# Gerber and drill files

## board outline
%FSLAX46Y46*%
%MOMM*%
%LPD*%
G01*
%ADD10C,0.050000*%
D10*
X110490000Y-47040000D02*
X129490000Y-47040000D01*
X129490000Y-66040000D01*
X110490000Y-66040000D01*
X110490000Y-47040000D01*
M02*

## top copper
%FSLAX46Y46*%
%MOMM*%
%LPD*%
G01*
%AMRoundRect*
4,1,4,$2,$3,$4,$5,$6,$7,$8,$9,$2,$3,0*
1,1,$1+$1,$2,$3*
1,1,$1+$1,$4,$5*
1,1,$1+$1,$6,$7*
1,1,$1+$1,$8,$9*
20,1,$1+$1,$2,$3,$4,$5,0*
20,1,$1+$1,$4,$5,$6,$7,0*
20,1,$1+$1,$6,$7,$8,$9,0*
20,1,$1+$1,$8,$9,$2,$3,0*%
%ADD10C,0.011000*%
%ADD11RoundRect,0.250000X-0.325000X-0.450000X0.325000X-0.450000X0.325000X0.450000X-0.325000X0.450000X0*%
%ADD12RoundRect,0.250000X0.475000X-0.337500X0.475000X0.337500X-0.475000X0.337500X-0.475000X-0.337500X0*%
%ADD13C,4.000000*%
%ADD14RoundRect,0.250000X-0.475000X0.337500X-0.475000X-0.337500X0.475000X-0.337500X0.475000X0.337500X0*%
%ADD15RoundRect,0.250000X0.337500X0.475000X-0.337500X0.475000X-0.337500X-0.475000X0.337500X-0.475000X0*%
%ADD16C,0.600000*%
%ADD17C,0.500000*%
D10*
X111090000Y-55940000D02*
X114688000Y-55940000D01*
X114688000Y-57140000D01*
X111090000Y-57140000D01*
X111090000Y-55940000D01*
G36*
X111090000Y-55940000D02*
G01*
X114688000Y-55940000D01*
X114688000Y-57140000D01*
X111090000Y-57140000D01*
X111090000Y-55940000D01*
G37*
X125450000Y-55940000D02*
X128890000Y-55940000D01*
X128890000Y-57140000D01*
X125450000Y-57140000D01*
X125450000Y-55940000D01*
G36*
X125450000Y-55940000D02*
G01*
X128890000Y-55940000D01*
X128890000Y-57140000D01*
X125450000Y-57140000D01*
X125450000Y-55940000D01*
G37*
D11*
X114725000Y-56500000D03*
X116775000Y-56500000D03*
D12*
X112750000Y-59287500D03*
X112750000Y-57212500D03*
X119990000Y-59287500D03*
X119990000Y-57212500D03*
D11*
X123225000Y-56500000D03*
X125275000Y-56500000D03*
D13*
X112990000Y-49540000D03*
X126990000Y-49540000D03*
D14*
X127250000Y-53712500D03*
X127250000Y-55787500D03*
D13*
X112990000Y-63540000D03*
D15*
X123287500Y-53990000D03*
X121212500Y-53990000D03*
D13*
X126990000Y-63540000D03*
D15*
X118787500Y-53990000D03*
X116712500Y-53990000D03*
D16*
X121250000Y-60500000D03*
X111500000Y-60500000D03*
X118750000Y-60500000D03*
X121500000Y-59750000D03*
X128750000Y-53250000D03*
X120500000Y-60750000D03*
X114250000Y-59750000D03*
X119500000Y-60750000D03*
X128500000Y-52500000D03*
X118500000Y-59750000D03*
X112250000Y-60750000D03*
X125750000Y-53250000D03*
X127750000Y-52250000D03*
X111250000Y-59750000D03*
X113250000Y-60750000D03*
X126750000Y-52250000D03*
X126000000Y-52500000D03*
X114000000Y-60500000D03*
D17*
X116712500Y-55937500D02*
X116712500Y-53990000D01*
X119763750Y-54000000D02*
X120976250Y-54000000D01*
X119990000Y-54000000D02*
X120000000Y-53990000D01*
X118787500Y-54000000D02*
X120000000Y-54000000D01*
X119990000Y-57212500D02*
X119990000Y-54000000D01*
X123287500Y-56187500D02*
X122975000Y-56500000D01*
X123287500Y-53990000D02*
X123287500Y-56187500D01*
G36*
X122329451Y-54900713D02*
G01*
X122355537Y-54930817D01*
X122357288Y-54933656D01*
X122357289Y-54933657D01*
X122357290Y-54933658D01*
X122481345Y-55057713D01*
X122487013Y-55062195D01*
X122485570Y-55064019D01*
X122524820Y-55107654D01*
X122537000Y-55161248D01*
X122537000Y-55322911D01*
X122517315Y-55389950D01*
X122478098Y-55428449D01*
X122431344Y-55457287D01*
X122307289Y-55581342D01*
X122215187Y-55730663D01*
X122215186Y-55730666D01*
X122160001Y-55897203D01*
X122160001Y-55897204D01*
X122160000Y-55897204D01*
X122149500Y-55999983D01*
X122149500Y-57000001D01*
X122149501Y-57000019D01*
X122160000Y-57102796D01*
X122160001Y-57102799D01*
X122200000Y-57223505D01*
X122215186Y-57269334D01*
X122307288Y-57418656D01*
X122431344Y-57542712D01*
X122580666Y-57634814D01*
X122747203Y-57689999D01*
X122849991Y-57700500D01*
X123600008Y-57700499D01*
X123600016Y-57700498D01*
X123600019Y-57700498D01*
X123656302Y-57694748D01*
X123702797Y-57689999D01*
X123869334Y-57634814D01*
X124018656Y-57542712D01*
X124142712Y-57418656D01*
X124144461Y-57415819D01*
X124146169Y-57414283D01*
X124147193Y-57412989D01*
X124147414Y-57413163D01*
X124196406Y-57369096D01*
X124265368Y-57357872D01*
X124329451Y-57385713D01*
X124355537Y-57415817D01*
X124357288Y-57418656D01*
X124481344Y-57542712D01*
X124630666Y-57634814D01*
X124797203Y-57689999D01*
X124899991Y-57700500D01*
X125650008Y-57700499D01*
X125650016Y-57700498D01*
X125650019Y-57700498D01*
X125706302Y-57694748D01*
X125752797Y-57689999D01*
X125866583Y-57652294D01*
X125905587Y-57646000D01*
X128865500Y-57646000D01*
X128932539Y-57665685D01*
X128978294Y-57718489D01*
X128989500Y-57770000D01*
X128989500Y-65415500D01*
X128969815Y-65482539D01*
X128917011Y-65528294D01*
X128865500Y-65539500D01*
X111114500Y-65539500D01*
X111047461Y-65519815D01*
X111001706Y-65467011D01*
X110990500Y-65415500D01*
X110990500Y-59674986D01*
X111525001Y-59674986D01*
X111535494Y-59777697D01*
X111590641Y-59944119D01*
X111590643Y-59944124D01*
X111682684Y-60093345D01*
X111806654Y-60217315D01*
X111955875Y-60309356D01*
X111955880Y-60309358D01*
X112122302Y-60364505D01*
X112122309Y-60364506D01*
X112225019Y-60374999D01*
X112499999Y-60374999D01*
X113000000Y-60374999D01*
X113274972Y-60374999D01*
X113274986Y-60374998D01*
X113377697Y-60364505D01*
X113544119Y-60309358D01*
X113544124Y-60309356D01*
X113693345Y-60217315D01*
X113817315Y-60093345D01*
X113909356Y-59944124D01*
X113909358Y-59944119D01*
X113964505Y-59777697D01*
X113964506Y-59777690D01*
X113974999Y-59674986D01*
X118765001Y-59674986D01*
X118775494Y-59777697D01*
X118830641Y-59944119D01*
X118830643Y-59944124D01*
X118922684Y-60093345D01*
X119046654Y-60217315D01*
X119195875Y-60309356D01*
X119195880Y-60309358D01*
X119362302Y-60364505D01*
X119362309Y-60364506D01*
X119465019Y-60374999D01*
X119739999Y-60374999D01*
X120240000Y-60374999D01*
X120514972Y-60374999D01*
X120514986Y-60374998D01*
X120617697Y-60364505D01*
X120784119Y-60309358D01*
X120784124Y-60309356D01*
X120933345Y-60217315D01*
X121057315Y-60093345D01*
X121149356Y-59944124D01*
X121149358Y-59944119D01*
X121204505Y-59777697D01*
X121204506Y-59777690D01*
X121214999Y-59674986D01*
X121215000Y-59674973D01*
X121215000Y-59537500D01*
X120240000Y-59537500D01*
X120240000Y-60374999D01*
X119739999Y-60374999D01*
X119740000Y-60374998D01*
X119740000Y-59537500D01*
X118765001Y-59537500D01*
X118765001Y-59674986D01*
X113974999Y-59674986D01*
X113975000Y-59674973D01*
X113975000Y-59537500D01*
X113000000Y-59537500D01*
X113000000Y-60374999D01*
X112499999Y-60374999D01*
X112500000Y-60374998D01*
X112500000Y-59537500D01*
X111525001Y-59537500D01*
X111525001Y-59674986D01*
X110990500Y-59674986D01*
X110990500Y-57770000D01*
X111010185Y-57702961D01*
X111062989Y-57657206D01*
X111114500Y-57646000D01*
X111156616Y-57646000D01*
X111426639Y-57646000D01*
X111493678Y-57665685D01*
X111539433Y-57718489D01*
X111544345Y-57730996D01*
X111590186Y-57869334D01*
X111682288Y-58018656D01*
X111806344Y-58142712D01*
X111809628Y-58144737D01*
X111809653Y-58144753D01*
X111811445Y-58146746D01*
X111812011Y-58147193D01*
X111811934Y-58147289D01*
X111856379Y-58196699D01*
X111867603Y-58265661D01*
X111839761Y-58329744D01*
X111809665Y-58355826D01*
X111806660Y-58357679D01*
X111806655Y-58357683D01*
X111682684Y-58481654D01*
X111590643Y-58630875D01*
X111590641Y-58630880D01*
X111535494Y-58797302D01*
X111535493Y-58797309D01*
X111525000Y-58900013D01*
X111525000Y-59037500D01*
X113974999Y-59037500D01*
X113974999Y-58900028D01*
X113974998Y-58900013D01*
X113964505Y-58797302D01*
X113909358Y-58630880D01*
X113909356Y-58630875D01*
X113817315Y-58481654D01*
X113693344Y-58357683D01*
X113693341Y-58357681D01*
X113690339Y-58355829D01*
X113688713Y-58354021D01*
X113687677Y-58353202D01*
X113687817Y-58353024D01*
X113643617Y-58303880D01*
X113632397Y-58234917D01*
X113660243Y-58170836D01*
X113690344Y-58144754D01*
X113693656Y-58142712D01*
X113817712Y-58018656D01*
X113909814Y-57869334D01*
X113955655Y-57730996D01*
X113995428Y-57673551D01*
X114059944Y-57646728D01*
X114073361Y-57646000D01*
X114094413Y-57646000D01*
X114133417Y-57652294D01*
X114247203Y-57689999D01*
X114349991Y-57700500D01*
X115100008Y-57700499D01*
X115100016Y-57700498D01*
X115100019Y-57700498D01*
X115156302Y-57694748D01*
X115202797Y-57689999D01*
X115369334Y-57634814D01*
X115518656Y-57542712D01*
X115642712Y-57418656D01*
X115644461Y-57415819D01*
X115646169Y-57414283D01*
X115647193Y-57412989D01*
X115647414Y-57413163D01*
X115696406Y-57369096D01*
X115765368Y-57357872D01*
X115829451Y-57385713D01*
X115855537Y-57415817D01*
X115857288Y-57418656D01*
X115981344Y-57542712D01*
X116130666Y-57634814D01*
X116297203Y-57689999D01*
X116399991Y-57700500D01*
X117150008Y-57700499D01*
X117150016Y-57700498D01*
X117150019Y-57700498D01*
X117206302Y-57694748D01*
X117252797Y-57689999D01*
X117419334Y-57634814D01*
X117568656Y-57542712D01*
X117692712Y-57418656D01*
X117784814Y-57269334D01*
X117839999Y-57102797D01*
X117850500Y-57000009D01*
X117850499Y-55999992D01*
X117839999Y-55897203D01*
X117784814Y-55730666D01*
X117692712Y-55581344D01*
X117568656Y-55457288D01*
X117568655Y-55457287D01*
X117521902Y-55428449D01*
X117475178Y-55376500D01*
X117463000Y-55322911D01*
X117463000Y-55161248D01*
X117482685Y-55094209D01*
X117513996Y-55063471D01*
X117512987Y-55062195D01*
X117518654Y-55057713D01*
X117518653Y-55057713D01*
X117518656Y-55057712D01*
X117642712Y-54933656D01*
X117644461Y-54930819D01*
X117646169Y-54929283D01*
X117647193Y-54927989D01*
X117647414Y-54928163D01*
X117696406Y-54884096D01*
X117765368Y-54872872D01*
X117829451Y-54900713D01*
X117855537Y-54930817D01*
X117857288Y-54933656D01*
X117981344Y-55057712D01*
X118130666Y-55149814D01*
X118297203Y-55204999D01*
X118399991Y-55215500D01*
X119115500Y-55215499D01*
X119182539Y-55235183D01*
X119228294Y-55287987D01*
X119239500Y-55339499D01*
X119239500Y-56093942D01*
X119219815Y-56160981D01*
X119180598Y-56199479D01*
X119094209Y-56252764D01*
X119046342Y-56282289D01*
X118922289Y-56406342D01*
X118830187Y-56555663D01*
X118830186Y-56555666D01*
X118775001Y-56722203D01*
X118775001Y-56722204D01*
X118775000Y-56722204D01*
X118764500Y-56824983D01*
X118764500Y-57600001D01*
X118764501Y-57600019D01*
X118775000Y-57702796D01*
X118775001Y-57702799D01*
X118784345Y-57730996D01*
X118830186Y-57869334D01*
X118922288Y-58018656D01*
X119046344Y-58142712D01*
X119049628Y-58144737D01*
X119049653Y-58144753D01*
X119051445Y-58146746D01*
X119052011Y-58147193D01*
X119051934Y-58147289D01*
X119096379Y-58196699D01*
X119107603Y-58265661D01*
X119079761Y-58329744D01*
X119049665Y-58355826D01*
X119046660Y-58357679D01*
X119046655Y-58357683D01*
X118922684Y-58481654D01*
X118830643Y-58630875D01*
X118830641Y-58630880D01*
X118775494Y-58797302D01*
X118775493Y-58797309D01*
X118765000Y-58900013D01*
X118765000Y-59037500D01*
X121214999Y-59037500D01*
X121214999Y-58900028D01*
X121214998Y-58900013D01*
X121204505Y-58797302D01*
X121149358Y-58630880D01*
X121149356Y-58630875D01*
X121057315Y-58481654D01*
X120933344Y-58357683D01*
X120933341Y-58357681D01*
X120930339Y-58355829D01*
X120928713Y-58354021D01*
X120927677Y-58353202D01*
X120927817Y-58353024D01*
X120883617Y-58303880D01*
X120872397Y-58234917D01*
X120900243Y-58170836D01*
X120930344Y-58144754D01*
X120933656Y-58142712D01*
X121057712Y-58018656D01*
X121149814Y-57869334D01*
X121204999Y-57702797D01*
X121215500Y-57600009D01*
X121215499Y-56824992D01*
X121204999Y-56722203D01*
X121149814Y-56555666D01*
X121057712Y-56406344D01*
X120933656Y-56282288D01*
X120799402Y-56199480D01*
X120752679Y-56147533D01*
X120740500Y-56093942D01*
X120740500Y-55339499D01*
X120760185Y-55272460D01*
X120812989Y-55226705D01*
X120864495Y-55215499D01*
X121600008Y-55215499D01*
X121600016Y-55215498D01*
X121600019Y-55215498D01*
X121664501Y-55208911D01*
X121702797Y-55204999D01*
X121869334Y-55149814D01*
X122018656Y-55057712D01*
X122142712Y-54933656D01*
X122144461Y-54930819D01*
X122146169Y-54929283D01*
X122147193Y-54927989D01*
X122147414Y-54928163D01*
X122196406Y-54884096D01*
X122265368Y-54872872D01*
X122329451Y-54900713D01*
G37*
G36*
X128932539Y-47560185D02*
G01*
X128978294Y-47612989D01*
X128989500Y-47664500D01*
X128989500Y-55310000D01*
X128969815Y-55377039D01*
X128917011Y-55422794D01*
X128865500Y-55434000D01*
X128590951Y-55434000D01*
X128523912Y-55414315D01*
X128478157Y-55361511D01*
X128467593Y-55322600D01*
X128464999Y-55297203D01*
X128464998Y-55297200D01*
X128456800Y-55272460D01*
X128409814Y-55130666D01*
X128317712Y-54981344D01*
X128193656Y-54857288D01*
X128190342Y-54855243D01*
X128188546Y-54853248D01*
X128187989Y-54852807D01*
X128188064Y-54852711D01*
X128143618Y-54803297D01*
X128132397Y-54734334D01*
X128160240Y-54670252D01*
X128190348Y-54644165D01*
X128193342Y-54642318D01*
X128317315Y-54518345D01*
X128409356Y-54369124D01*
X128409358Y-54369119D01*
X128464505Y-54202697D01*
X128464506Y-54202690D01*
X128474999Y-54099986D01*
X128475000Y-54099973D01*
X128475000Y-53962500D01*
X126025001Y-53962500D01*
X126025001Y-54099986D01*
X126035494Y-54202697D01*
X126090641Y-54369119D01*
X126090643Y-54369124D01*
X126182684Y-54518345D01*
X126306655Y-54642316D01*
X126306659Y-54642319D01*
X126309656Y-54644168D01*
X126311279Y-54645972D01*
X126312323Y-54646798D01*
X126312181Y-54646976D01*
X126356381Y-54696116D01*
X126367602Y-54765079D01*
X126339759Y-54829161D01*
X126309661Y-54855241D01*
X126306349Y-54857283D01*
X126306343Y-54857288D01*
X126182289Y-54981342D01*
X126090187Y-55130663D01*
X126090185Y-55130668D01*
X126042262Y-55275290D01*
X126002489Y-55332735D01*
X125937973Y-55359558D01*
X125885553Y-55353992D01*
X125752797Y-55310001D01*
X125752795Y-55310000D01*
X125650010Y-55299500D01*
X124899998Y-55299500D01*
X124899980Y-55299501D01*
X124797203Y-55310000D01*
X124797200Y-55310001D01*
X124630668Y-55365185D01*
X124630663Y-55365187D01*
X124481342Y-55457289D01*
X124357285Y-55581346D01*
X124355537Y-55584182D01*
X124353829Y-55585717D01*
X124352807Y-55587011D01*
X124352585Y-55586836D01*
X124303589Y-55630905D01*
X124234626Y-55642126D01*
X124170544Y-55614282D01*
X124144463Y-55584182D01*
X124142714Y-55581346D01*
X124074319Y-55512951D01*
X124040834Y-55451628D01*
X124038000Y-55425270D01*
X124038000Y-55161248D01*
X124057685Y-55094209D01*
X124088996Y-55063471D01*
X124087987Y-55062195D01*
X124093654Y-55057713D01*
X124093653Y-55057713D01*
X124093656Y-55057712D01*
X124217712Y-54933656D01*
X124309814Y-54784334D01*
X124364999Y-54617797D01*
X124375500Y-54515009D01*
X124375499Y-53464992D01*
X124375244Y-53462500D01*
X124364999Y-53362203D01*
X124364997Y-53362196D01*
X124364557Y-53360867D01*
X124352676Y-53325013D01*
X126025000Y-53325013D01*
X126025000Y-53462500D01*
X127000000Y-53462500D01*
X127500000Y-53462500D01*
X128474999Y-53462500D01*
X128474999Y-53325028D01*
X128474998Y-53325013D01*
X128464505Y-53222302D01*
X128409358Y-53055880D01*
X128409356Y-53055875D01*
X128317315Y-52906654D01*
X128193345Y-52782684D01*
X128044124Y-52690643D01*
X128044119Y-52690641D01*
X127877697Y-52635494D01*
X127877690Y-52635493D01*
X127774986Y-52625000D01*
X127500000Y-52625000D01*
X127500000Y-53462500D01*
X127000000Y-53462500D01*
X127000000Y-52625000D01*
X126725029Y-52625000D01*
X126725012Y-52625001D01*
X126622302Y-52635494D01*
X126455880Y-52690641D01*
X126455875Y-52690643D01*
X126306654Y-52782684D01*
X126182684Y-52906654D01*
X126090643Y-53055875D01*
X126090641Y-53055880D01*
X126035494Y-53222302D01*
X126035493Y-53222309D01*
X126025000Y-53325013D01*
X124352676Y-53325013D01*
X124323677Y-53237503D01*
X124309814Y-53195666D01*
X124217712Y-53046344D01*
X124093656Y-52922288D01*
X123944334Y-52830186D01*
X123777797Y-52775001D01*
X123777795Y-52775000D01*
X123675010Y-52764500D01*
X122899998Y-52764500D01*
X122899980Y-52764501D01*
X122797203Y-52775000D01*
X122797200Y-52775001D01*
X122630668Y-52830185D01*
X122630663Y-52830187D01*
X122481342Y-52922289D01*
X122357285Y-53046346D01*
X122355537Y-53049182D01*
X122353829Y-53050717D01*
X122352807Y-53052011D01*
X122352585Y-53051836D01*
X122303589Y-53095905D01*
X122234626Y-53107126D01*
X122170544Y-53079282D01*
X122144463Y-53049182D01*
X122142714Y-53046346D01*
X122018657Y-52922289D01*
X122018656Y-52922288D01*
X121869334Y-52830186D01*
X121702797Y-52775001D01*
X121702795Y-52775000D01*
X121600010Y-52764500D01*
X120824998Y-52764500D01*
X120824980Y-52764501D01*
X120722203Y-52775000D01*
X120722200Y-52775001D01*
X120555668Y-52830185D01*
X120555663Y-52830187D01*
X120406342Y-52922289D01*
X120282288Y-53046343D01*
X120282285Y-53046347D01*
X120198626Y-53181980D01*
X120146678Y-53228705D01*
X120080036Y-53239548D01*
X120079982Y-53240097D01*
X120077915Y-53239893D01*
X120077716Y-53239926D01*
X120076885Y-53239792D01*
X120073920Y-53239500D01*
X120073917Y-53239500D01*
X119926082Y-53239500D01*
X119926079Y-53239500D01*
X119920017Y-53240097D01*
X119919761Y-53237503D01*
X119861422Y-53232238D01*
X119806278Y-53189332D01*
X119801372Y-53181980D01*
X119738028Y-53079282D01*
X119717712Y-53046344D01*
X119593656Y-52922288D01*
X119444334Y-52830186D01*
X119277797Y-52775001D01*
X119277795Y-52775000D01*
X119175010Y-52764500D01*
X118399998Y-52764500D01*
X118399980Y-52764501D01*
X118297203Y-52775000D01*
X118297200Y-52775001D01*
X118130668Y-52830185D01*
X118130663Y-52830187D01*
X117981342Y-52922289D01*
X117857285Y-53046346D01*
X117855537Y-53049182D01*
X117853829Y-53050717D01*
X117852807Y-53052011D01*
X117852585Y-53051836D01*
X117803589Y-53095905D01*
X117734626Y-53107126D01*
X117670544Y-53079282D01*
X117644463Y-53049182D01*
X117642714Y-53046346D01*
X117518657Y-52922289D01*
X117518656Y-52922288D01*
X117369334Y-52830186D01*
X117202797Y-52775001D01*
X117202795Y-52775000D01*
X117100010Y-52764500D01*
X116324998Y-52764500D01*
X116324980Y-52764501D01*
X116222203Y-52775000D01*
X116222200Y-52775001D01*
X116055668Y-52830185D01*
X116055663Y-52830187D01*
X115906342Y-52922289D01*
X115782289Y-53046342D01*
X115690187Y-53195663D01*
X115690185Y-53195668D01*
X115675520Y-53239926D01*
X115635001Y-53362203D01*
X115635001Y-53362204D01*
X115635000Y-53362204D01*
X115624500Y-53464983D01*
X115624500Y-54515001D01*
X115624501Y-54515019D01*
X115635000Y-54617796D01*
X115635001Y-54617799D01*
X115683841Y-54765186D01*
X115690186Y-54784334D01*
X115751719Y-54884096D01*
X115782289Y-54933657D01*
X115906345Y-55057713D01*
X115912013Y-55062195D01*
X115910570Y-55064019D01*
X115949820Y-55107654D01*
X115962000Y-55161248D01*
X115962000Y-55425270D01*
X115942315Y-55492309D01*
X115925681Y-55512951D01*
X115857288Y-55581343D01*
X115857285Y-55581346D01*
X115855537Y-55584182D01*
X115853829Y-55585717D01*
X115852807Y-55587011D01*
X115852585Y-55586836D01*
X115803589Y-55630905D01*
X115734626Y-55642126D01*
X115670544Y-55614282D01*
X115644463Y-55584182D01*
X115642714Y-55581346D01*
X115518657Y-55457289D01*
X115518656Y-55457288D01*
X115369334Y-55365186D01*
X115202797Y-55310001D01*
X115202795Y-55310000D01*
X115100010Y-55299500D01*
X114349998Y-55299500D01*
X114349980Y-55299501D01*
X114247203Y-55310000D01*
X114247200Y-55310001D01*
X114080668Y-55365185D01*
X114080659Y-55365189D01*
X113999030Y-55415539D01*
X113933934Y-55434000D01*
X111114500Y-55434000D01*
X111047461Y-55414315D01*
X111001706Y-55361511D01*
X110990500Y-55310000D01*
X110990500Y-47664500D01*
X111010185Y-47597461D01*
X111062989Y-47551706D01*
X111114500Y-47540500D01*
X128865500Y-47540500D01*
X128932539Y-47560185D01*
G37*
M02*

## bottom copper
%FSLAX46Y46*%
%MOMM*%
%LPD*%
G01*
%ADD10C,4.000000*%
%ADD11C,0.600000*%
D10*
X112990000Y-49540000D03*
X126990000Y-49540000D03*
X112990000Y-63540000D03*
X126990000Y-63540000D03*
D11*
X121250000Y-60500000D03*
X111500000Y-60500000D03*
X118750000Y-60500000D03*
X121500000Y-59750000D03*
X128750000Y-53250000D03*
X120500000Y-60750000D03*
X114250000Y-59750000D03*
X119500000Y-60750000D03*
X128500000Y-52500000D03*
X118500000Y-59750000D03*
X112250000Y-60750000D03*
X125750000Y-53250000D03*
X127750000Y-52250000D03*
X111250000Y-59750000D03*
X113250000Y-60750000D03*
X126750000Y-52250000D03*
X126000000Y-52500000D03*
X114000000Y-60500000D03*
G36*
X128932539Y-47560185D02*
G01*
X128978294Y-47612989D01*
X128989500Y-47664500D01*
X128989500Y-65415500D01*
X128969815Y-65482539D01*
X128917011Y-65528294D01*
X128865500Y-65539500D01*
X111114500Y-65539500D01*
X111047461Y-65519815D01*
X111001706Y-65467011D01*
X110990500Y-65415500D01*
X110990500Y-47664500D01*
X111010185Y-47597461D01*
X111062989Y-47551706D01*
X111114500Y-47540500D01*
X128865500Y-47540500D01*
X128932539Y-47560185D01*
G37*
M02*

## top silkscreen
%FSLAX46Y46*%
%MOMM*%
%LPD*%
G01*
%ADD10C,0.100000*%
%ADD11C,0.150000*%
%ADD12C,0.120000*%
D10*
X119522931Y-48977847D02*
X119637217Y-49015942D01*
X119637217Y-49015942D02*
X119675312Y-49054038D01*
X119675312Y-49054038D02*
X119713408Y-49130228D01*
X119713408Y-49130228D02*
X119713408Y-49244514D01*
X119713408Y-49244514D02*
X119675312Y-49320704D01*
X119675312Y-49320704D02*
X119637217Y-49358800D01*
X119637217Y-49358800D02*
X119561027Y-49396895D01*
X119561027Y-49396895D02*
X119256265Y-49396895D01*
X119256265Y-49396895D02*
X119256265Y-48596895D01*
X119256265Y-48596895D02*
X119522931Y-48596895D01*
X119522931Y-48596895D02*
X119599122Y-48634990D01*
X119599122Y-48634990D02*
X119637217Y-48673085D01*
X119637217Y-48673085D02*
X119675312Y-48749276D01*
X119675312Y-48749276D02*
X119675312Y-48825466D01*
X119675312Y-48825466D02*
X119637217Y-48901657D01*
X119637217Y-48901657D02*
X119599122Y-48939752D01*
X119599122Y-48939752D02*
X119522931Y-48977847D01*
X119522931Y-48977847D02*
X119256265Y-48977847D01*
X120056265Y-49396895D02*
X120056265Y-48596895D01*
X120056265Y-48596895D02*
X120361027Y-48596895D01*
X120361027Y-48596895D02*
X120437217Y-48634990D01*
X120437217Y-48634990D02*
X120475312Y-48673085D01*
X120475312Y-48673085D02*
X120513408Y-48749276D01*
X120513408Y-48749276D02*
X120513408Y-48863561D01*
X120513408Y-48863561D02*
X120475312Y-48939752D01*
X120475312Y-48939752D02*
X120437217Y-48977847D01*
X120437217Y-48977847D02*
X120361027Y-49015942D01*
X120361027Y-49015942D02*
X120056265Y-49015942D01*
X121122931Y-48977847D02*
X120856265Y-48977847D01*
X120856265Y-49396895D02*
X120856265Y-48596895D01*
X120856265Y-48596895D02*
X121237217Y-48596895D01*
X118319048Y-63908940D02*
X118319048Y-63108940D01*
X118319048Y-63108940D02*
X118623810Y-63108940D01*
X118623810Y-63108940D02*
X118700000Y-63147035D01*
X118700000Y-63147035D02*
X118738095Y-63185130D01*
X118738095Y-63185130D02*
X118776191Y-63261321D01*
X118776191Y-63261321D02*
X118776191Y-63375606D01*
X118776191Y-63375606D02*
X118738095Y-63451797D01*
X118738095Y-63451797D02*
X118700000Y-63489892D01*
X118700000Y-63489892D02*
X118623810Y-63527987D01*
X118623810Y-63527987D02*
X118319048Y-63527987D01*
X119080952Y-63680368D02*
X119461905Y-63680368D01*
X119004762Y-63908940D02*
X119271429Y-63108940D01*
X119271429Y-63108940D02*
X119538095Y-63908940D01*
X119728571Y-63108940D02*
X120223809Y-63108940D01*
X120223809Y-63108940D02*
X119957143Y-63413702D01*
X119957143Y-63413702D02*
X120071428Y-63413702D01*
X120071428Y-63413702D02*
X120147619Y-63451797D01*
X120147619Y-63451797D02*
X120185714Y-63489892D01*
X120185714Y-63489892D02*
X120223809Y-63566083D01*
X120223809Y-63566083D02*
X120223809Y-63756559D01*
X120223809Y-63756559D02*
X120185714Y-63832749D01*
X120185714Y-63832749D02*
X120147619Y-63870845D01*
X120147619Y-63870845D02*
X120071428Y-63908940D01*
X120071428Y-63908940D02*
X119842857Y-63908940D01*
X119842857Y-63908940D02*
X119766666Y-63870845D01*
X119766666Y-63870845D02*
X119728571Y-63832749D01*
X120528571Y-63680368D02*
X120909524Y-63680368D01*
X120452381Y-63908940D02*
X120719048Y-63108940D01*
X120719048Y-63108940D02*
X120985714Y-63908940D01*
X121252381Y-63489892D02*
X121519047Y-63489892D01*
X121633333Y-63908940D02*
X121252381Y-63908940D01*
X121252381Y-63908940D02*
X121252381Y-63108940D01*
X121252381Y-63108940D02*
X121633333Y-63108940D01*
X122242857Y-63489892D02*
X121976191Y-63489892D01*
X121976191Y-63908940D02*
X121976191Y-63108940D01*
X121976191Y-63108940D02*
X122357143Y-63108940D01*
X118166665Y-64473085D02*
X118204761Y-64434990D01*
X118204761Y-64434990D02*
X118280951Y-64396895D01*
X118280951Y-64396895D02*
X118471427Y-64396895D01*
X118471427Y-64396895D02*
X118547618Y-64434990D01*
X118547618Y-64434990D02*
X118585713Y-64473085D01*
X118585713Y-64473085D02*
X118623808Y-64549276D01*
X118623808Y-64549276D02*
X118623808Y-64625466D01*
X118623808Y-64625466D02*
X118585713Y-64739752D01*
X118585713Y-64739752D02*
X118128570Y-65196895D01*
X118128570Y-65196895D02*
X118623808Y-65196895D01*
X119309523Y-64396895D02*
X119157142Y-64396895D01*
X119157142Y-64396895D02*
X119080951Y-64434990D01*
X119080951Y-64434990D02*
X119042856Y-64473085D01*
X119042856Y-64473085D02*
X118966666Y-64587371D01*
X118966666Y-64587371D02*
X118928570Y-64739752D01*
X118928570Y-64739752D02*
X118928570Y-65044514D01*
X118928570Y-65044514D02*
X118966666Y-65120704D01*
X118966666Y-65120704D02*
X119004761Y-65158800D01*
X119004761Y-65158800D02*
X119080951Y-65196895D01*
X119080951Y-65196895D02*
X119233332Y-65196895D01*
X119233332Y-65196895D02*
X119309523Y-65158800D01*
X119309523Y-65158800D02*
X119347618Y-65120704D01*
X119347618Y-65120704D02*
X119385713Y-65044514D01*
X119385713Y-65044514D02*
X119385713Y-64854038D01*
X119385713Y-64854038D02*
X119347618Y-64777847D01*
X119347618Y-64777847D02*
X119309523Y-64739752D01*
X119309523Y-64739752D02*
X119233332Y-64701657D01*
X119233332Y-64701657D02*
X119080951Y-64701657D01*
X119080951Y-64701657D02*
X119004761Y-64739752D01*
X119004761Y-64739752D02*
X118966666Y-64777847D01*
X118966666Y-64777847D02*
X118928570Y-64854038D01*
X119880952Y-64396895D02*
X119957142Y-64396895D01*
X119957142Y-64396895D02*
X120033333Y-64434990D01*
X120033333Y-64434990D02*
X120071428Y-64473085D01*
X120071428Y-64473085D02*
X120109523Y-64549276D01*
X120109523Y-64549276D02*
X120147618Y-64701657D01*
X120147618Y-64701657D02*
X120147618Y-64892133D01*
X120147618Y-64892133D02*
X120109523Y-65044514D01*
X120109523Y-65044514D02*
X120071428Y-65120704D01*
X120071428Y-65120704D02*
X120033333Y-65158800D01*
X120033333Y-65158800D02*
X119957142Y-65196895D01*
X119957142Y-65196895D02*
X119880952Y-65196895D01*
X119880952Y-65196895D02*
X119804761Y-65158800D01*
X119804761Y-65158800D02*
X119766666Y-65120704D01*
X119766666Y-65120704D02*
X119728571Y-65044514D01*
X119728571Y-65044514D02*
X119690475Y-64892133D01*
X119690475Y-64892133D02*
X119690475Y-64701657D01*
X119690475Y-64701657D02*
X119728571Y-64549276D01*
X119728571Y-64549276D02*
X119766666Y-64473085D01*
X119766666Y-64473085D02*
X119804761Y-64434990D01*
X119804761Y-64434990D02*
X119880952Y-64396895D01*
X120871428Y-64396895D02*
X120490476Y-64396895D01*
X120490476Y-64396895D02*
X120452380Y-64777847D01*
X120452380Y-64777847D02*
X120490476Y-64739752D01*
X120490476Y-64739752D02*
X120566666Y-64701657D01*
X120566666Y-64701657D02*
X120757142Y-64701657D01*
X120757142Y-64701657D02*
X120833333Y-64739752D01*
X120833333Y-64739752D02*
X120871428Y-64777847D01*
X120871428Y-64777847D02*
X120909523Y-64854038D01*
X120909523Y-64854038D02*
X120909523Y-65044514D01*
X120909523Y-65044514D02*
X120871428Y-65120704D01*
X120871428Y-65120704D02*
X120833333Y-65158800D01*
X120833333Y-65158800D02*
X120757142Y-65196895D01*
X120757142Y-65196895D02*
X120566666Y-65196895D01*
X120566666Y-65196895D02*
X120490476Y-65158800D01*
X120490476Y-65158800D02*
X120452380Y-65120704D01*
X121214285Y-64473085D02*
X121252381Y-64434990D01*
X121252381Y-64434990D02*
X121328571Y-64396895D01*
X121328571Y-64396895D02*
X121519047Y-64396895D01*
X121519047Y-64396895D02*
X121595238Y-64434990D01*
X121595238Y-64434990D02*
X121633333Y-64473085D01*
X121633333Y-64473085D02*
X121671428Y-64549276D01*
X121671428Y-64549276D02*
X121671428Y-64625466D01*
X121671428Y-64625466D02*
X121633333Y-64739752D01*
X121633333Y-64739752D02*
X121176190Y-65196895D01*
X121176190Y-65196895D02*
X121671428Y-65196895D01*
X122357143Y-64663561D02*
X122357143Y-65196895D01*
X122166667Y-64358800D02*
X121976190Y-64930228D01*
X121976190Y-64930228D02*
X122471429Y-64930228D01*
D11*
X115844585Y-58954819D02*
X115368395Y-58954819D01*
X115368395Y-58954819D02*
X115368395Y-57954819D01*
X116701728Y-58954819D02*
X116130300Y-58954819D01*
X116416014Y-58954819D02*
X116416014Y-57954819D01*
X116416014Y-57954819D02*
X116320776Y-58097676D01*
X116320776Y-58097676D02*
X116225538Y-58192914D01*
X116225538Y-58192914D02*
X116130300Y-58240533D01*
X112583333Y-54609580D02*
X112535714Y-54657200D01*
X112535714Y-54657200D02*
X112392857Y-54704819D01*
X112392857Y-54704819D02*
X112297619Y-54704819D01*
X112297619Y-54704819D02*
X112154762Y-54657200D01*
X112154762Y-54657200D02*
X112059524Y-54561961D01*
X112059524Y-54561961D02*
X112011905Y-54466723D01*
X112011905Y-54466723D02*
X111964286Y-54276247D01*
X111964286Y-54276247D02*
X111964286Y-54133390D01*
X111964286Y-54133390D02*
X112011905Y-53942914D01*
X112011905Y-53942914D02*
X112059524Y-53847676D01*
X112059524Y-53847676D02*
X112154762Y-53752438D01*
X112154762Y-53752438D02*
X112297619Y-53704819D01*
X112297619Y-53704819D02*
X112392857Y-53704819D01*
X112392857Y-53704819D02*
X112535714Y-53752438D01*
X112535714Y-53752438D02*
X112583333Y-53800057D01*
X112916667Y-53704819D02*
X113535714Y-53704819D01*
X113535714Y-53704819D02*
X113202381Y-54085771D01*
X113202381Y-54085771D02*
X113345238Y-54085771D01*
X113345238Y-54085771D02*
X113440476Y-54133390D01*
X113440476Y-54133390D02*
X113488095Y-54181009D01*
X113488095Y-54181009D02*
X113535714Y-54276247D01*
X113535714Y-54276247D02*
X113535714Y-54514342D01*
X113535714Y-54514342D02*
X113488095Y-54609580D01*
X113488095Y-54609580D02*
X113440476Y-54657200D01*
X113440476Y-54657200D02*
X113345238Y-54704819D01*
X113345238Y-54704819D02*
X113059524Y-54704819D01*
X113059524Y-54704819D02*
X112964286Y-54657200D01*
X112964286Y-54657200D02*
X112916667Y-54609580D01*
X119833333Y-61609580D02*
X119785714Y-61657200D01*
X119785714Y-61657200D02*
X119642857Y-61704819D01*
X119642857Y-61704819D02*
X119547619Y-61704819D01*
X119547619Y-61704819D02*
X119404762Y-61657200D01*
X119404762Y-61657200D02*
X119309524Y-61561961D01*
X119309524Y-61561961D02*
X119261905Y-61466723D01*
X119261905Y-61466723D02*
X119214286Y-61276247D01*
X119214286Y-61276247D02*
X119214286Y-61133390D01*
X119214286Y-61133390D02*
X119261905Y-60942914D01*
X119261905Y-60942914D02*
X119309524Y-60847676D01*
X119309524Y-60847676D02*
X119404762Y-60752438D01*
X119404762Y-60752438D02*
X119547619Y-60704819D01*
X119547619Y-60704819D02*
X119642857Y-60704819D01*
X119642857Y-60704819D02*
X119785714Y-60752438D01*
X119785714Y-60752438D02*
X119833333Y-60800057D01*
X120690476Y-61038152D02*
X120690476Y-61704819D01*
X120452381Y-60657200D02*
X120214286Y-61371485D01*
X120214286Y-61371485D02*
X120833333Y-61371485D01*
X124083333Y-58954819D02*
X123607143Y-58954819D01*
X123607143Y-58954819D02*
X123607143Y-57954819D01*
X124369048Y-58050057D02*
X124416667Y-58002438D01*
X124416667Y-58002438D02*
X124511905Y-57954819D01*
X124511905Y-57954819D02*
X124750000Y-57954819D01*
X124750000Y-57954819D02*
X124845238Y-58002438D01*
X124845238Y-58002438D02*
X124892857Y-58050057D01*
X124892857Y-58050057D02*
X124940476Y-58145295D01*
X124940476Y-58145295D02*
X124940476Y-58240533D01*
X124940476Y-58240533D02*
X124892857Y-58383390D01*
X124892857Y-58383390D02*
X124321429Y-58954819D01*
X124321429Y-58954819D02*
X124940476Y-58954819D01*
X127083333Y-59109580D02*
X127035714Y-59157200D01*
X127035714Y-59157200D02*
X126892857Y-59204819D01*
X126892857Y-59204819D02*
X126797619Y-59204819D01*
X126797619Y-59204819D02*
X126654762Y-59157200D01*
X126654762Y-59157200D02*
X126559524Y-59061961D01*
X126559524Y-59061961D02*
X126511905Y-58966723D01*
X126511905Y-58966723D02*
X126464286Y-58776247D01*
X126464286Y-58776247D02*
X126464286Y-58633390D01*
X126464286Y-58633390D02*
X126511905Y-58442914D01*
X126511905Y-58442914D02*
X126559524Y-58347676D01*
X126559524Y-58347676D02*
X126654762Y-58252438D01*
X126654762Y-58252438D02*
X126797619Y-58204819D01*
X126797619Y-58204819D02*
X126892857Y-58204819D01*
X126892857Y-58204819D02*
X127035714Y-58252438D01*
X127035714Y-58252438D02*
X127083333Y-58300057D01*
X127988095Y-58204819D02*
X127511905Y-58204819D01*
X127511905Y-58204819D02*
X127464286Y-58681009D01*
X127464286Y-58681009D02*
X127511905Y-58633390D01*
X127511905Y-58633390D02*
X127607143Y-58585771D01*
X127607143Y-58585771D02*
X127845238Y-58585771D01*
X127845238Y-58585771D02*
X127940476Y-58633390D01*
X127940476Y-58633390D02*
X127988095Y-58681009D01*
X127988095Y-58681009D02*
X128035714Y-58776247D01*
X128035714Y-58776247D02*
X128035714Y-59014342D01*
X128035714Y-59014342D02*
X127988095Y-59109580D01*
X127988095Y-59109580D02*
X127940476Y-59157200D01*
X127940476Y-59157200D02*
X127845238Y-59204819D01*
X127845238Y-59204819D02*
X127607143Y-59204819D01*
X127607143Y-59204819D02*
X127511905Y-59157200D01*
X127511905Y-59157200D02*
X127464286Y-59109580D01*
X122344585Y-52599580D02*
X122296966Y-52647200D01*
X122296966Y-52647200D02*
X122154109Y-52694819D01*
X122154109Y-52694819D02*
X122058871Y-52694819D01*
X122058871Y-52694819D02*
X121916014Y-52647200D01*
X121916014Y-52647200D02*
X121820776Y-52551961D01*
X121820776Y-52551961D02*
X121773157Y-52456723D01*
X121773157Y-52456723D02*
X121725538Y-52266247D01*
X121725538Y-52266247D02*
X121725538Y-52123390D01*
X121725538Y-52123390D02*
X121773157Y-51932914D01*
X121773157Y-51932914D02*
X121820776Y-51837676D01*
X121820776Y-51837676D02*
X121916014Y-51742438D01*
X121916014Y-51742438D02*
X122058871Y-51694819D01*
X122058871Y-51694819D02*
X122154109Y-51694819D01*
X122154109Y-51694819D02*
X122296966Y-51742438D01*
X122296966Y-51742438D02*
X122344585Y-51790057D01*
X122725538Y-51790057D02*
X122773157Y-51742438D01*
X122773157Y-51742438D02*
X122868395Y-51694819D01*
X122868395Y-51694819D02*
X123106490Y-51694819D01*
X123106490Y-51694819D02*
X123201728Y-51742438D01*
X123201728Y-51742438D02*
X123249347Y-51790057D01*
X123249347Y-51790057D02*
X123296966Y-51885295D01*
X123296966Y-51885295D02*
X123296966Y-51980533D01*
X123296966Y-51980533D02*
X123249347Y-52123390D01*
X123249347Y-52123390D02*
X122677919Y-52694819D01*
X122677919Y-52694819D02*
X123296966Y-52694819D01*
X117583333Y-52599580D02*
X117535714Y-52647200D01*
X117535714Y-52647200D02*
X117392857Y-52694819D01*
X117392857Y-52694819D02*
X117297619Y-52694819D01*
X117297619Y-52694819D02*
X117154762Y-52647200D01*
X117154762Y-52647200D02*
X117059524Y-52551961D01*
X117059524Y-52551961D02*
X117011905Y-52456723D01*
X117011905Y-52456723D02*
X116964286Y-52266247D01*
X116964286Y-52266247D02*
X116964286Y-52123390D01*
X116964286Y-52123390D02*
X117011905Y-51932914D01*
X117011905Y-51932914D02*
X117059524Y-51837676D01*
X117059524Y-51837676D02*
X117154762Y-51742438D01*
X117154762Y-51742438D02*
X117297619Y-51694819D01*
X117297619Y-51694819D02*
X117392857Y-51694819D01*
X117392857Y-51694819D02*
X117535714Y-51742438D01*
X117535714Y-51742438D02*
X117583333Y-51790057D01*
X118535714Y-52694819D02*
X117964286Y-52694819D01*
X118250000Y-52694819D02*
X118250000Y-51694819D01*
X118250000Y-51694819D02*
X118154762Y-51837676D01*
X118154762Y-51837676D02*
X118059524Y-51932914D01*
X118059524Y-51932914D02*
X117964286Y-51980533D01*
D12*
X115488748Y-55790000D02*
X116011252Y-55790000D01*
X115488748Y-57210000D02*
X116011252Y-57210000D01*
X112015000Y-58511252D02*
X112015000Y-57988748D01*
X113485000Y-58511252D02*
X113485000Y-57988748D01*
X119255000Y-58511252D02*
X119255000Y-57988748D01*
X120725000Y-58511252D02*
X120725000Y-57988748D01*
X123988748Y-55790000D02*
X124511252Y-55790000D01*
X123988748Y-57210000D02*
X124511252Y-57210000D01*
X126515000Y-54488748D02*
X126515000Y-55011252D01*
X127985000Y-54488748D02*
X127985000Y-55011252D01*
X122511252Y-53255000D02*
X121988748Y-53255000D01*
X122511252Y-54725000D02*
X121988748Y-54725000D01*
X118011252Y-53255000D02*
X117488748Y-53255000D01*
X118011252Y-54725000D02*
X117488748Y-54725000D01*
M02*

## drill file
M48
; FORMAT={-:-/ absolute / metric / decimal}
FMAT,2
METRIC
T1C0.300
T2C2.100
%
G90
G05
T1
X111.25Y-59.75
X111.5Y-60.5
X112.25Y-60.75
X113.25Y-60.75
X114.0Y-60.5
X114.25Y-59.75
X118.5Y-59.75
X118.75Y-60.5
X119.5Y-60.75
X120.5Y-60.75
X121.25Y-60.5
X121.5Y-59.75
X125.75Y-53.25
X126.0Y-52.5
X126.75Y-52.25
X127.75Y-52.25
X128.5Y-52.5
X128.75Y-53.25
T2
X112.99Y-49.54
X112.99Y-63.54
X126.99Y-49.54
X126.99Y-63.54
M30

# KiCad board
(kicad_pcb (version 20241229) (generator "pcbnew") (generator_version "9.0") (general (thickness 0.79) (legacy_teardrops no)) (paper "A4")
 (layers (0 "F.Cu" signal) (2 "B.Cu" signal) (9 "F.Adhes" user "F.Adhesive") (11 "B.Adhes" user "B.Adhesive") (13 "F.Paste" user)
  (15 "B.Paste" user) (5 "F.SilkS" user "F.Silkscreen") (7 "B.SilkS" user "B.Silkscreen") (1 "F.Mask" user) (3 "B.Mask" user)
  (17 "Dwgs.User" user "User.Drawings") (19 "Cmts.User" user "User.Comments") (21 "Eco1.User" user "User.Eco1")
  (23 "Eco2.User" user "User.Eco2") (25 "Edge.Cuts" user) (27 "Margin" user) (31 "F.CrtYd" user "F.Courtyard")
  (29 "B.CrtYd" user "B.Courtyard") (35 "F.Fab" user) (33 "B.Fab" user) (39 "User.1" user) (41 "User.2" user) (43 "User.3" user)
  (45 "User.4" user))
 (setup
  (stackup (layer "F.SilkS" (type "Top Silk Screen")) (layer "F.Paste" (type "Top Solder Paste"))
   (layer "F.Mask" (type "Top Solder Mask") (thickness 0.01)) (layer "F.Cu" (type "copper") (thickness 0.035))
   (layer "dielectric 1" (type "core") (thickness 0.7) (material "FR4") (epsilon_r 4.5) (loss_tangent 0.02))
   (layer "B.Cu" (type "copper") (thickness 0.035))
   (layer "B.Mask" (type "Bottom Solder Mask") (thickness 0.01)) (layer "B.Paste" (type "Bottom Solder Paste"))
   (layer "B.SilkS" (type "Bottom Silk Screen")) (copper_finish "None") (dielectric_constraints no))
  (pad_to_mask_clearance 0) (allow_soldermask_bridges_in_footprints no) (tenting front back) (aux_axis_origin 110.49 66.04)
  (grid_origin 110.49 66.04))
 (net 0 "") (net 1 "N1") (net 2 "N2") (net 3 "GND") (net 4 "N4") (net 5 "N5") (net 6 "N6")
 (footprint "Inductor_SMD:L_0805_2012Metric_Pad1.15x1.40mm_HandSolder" (layer "F.Cu") (at 115.75 56.5)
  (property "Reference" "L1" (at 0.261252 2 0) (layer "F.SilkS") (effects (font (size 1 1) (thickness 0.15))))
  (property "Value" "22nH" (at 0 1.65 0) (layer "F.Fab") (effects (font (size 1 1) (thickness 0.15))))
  (fp_line (start -0.261252 -0.71) (end 0.261252 -0.71) (stroke (width 0.12) (type solid)) (layer "F.SilkS"))
  (fp_line (start -0.261252 0.71) (end 0.261252 0.71) (stroke (width 0.12) (type solid)) (layer "F.SilkS"))
  (pad "1" smd roundrect (at -1.025 0) (size 1.15 1.4) (layers "F.Cu" "F.Mask" "F.Paste") (roundrect_rratio 0.217391) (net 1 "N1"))
  (pad "2" smd roundrect (at 1.025 0) (size 1.15 1.4) (layers "F.Cu" "F.Mask" "F.Paste") (roundrect_rratio 0.217391) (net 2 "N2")))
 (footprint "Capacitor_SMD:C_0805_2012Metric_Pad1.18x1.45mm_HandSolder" (layer "F.Cu") (at 112.75 58.25 90)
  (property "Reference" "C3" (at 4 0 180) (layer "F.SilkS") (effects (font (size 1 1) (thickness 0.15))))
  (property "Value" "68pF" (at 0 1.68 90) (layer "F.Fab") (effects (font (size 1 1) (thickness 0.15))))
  (fp_line (start -0.261252 -0.735) (end 0.261252 -0.735) (stroke (width 0.12) (type solid)) (layer "F.SilkS"))
  (fp_line (start -0.261252 0.735) (end 0.261252 0.735) (stroke (width 0.12) (type solid)) (layer "F.SilkS"))
  (pad "1" smd roundrect (at -1.0375 0 90) (size 1.175 1.45) (layers "F.Cu" "F.Mask" "F.Paste") (roundrect_rratio 0.212766) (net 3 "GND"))
  (pad "2" smd roundrect (at 1.0375 0 90) (size 1.175 1.45) (layers "F.Cu" "F.Mask" "F.Paste") (roundrect_rratio 0.212766) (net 1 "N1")))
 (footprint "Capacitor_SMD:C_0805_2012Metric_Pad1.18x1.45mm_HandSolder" (layer "F.Cu") (at 119.99 58.25 90)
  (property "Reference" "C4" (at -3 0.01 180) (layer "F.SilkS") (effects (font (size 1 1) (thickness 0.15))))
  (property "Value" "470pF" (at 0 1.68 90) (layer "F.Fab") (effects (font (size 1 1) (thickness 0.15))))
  (fp_line (start -0.261252 -0.735) (end 0.261252 -0.735) (stroke (width 0.12) (type solid)) (layer "F.SilkS"))
  (fp_line (start -0.261252 0.735) (end 0.261252 0.735) (stroke (width 0.12) (type solid)) (layer "F.SilkS"))
  (pad "1" smd roundrect (at -1.0375 0 90) (size 1.175 1.45) (layers "F.Cu" "F.Mask" "F.Paste") (roundrect_rratio 0.212766) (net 3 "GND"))
  (pad "2" smd roundrect (at 1.0375 0 90) (size 1.175 1.45) (layers "F.Cu" "F.Mask" "F.Paste") (roundrect_rratio 0.212766) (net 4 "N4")))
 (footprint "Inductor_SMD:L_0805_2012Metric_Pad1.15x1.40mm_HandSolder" (layer "F.Cu") (at 124.25 56.5)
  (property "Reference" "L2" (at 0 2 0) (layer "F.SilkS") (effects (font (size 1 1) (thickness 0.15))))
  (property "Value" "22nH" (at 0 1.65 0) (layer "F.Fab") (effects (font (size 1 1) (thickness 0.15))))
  (fp_line (start -0.261252 -0.71) (end 0.261252 -0.71) (stroke (width 0.12) (type solid)) (layer "F.SilkS"))
  (fp_line (start -0.261252 0.71) (end 0.261252 0.71) (stroke (width 0.12) (type solid)) (layer "F.SilkS"))
  (pad "1" smd roundrect (at -1.025 0) (size 1.15 1.4) (layers "F.Cu" "F.Mask" "F.Paste") (roundrect_rratio 0.217391) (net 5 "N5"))
  (pad "2" smd roundrect (at 1.025 0) (size 1.15 1.4) (layers "F.Cu" "F.Mask" "F.Paste") (roundrect_rratio 0.217391) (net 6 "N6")))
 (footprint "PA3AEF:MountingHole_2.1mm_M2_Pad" (layer "F.Cu") (at 112.99 49.54)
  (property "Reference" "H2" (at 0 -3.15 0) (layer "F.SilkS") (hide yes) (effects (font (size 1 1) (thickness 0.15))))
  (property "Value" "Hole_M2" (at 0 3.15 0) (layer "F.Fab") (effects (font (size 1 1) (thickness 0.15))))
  (pad "1" thru_hole circle (at 0 0) (size 4 4) (drill 2.1) (layers "*.Cu" "*.Mask") (remove_unused_layers no) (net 3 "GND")
   (zone_connect 2)))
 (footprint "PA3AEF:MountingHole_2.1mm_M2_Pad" (layer "F.Cu") (at 126.99 49.54)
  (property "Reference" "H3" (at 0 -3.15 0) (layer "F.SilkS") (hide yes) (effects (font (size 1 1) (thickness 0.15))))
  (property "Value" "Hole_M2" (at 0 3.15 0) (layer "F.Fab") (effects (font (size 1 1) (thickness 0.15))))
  (pad "1" thru_hole circle (at 0 0) (size 4 4) (drill 2.1) (layers "*.Cu" "*.Mask") (remove_unused_layers no) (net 3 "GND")
   (zone_connect 2)))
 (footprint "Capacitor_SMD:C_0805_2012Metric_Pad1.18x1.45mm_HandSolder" (layer "F.Cu") (at 127.25 54.75 -90)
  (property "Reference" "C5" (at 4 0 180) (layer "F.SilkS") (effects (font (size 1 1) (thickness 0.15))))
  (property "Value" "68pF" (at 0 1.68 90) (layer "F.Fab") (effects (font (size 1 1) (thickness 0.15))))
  (fp_line (start -0.261252 0.735) (end 0.261252 0.735) (stroke (width 0.12) (type solid)) (layer "F.SilkS"))
  (fp_line (start -0.261252 -0.735) (end 0.261252 -0.735) (stroke (width 0.12) (type solid)) (layer "F.SilkS"))
  (pad "1" smd roundrect (at -1.0375 0 270) (size 1.175 1.45) (layers "F.Cu" "F.Mask" "F.Paste") (roundrect_rratio 0.212766) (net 3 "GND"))
  (pad "2" smd roundrect (at 1.0375 0 270) (size 1.175 1.45) (layers "F.Cu" "F.Mask" "F.Paste") (roundrect_rratio 0.212766) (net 6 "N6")))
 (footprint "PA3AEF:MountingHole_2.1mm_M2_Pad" (layer "F.Cu") (at 112.99 63.54)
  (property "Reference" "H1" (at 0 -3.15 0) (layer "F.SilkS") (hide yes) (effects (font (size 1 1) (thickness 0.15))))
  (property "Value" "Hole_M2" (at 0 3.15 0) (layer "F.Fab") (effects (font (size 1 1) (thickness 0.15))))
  (pad "1" thru_hole circle (at 0 0) (size 4 4) (drill 2.1) (layers "*.Cu" "*.Mask") (remove_unused_layers no) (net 3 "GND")
   (zone_connect 2)))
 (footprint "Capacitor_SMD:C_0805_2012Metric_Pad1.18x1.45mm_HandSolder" (layer "F.Cu") (at 122.25 53.99 180)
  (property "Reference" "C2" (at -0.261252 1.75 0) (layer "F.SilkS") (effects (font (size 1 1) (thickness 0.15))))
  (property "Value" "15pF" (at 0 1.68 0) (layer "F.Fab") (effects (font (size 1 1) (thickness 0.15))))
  (fp_line (start -0.261252 0.735) (end 0.261252 0.735) (stroke (width 0.12) (type solid)) (layer "F.SilkS"))
  (fp_line (start -0.261252 -0.735) (end 0.261252 -0.735) (stroke (width 0.12) (type solid)) (layer "F.SilkS"))
  (pad "1" smd roundrect (at -1.0375 0 180) (size 1.175 1.45) (layers "F.Cu" "F.Mask" "F.Paste") (roundrect_rratio 0.212766) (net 5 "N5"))
  (pad "2" smd roundrect (at 1.0375 0 180) (size 1.175 1.45) (layers "F.Cu" "F.Mask" "F.Paste") (roundrect_rratio 0.212766) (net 4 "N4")))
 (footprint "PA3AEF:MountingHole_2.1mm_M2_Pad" (layer "F.Cu") (at 126.99 63.54)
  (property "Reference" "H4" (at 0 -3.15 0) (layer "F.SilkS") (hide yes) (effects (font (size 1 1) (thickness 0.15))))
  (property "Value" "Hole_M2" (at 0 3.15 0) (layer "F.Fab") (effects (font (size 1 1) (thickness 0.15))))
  (pad "1" thru_hole circle (at 0 0) (size 4 4) (drill 2.1) (layers "*.Cu" "*.Mask") (remove_unused_layers no) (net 3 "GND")
   (zone_connect 2)))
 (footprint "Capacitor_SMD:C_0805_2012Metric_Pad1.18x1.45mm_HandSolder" (layer "F.Cu") (at 117.75 53.99 180)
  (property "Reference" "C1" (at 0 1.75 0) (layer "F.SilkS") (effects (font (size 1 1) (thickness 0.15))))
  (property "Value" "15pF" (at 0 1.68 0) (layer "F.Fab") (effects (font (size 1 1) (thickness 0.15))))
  (fp_line (start -0.261252 0.735) (end 0.261252 0.735) (stroke (width 0.12) (type solid)) (layer "F.SilkS"))
  (fp_line (start -0.261252 -0.735) (end 0.261252 -0.735) (stroke (width 0.12) (type solid)) (layer "F.SilkS"))
  (pad "1" smd roundrect (at -1.0375 0 180) (size 1.175 1.45) (layers "F.Cu" "F.Mask" "F.Paste") (roundrect_rratio 0.212766) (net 4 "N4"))
  (pad "2" smd roundrect (at 1.0375 0 180) (size 1.175 1.45) (layers "F.Cu" "F.Mask" "F.Paste") (roundrect_rratio 0.212766) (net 2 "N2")))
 (gr_rect (start 111.09 55.94) (end 114.688 57.14) (stroke (width 0.011) (type solid)) (fill yes) (layer "F.Cu") (net 1))
 (gr_rect (start 125.45 55.94) (end 128.89 57.14) (stroke (width 0.011) (type solid)) (fill yes) (layer "F.Cu") (net 6))
 (gr_rect (start 110.49 47.04) (end 129.49 66.04) (stroke (width 0.05) (type solid)) (fill no) (layer "Edge.Cuts"))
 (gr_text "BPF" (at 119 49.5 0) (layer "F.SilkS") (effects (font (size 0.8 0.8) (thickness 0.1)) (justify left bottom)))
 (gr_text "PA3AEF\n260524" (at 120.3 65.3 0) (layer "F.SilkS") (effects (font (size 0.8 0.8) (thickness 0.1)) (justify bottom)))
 (via (at 121.25 60.5) (size 0.6) (drill 0.3) (layers "F.Cu" "B.Cu") (free yes) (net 3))
 (via (at 111.5 60.5) (size 0.6) (drill 0.3) (layers "F.Cu" "B.Cu") (free yes) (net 3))
 (via (at 118.75 60.5) (size 0.6) (drill 0.3) (layers "F.Cu" "B.Cu") (free yes) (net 3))
 (via (at 121.5 59.75) (size 0.6) (drill 0.3) (layers "F.Cu" "B.Cu") (free yes) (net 3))
 (via (at 128.75 53.25) (size 0.6) (drill 0.3) (layers "F.Cu" "B.Cu") (free yes) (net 3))
 (via (at 120.5 60.75) (size 0.6) (drill 0.3) (layers "F.Cu" "B.Cu") (free yes) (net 3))
 (via (at 114.25 59.75) (size 0.6) (drill 0.3) (layers "F.Cu" "B.Cu") (free yes) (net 3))
 (via (at 119.5 60.75) (size 0.6) (drill 0.3) (layers "F.Cu" "B.Cu") (free yes) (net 3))
 (via (at 128.5 52.5) (size 0.6) (drill 0.3) (layers "F.Cu" "B.Cu") (free yes) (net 3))
 (via (at 118.5 59.75) (size 0.6) (drill 0.3) (layers "F.Cu" "B.Cu") (free yes) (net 3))
 (via (at 112.25 60.75) (size 0.6) (drill 0.3) (layers "F.Cu" "B.Cu") (free yes) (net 3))
 (via (at 125.75 53.25) (size 0.6) (drill 0.3) (layers "F.Cu" "B.Cu") (free yes) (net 3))
 (via (at 127.75 52.25) (size 0.6) (drill 0.3) (layers "F.Cu" "B.Cu") (free yes) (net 3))
 (via (at 111.25 59.75) (size 0.6) (drill 0.3) (layers "F.Cu" "B.Cu") (free yes) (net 3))
 (via (at 113.25 60.75) (size 0.6) (drill 0.3) (layers "F.Cu" "B.Cu") (free yes) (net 3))
 (via (at 126.75 52.25) (size 0.6) (drill 0.3) (layers "F.Cu" "B.Cu") (free yes) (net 3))
 (via (at 126 52.5) (size 0.6) (drill 0.3) (layers "F.Cu" "B.Cu") (free yes) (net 3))
 (via (at 114 60.5) (size 0.6) (drill 0.3) (layers "F.Cu" "B.Cu") (free yes) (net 3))
 (segment (start 116.7125 55.9375) (end 116.7125 53.99) (width 0.5) (layer "F.Cu") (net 2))
 (segment (start 119.76375 54) (end 120.97625 54) (width 0.5) (layer "F.Cu") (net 4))
 (segment (start 119.99 54) (end 120 53.99) (width 0.5) (layer "F.Cu") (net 4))
 (segment (start 118.7875 54) (end 120 54) (width 0.5) (layer "F.Cu") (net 4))
 (segment (start 119.99 57.2125) (end 119.99 54) (width 0.5) (layer "F.Cu") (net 4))
 (segment (start 123.2875 56.1875) (end 122.975 56.5) (width 0.5) (layer "F.Cu") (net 5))
 (segment (start 123.2875 53.99) (end 123.2875 56.1875) (width 0.5) (layer "F.Cu") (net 5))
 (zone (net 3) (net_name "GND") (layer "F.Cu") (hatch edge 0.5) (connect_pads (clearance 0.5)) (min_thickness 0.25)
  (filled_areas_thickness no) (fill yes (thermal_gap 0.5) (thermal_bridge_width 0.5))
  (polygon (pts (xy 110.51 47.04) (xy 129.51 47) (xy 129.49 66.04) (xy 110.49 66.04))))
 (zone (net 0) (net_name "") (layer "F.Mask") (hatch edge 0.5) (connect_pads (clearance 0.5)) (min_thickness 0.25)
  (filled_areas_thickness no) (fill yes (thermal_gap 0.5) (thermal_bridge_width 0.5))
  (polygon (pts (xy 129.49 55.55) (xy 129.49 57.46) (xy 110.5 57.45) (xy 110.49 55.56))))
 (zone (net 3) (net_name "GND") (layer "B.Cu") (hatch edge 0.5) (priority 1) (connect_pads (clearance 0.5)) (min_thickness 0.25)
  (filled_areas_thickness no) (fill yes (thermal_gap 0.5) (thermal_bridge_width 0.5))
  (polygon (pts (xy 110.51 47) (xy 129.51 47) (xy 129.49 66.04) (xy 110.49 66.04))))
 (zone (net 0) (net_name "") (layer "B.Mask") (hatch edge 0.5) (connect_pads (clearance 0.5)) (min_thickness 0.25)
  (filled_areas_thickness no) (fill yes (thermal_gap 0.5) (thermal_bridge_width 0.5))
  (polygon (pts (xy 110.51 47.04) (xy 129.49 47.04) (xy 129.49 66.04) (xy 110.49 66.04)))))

